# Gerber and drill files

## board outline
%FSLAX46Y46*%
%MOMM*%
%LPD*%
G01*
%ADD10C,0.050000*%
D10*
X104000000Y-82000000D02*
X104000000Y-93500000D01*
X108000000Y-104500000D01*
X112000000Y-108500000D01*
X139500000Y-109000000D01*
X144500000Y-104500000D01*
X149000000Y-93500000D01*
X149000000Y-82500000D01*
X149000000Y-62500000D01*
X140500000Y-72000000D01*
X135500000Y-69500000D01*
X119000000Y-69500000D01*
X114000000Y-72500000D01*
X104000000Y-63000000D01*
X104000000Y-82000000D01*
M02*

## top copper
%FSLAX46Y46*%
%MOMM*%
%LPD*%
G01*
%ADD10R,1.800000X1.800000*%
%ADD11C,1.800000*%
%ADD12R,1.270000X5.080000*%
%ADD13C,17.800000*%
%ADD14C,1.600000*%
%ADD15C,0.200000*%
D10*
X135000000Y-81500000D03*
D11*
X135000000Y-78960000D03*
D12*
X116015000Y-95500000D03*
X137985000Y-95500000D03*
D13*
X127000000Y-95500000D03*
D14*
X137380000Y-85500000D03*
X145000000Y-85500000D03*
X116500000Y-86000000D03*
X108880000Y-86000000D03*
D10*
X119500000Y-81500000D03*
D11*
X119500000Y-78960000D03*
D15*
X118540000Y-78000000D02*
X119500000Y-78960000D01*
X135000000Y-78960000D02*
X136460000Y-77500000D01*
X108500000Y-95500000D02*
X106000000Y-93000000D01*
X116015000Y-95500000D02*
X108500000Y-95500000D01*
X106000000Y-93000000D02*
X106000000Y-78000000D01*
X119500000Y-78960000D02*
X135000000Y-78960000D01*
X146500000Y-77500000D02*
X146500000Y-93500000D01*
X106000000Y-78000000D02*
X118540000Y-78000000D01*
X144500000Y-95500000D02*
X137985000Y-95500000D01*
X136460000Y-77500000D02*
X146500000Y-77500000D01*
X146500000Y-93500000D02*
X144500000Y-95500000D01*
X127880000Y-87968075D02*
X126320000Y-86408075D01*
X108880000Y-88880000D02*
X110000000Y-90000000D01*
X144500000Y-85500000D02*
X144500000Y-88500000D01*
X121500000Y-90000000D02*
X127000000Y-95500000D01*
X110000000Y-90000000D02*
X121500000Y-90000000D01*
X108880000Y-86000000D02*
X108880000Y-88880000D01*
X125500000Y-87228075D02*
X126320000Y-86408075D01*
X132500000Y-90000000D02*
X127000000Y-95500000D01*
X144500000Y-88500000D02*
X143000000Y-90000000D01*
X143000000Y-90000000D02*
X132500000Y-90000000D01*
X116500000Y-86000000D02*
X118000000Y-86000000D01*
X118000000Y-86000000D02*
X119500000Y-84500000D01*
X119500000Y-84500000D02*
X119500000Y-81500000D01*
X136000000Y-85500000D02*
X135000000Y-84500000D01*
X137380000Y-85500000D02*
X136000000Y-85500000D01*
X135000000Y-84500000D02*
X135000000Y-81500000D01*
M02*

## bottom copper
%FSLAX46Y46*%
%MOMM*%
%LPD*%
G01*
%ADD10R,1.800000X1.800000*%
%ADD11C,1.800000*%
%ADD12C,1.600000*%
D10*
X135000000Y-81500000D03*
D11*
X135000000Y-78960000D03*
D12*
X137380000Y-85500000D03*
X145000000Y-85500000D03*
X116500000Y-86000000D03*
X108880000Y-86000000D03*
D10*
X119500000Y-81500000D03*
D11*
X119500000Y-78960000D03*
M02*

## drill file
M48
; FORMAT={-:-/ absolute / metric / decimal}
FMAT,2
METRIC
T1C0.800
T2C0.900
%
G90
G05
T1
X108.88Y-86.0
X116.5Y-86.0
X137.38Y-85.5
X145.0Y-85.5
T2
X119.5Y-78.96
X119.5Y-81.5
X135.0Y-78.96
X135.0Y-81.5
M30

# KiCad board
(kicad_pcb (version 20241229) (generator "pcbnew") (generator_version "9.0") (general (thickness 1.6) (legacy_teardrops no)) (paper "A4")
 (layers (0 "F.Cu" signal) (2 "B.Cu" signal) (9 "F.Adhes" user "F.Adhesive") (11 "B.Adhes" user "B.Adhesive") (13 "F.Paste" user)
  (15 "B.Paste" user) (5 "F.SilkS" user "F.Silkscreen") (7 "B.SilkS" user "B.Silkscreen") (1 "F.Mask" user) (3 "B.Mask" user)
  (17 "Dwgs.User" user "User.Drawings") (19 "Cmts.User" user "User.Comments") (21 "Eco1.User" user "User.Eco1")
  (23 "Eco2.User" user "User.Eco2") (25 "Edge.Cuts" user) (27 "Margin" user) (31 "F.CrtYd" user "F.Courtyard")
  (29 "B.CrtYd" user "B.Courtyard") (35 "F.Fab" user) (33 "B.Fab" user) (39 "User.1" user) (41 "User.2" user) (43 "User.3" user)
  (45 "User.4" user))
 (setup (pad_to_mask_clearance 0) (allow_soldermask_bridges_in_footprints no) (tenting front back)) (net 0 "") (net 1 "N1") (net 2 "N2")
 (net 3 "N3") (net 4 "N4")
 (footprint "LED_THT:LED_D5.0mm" (layer "F.Cu") (at 135 81.5 90)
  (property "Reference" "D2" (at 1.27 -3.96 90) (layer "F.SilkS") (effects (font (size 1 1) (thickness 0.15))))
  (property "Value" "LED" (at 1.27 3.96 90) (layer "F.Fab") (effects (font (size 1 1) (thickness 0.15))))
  (pad "1" thru_hole rect (at 0 0 90) (size 1.8 1.8) (drill 0.9) (layers "*.Cu" "*.Mask") (remove_unused_layers no) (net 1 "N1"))
  (pad "2" thru_hole circle (at 2.54 0 90) (size 1.8 1.8) (drill 0.9) (layers "*.Cu" "*.Mask") (remove_unused_layers no) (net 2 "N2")))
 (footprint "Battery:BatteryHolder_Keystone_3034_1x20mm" (layer "F.Cu") (at 127 95.5)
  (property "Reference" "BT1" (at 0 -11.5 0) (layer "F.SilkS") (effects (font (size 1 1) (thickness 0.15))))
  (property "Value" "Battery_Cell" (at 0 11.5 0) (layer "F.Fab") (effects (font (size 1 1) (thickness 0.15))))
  (pad "1" smd rect (at -10.985 0) (size 1.27 5.08) (layers "F.Cu" "F.Mask" "F.Paste") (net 2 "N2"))
  (pad "1" smd rect (at 10.985 0) (size 1.27 5.08) (layers "F.Cu" "F.Mask" "F.Paste") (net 2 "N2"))
  (pad "2" smd circle (at 0 0) (size 17.8 17.8) (layers "F.Cu" "F.Mask") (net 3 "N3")))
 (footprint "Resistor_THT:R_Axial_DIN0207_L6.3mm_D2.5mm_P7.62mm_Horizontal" (layer "F.Cu") (at 137.38 85.5)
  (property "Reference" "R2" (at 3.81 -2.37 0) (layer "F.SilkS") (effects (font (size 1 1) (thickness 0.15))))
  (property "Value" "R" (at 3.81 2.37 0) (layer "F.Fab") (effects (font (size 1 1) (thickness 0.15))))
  (pad "1" thru_hole circle (at 0 0) (size 1.6 1.6) (drill 0.8) (layers "*.Cu" "*.Mask") (remove_unused_layers no) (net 1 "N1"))
  (pad "2" thru_hole circle (at 7.62 0) (size 1.6 1.6) (drill 0.8) (layers "*.Cu" "*.Mask") (remove_unused_layers no) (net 3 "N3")))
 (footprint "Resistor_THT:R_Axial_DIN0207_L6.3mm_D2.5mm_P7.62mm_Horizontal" (layer "F.Cu") (at 116.5 86 180)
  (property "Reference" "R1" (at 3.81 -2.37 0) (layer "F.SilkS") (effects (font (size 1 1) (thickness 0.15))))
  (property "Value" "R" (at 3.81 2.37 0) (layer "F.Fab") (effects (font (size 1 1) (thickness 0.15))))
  (pad "1" thru_hole circle (at 0 0 180) (size 1.6 1.6) (drill 0.8) (layers "*.Cu" "*.Mask") (remove_unused_layers no) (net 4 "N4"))
  (pad "2" thru_hole circle (at 7.62 0 180) (size 1.6 1.6) (drill 0.8) (layers "*.Cu" "*.Mask") (remove_unused_layers no) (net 3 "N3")))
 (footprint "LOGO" (layer "F.Cu") (at 146 73)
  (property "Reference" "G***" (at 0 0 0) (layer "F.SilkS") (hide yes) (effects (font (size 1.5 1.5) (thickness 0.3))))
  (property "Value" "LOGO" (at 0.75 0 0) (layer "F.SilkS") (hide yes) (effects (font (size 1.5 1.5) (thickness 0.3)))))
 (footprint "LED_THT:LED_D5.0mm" (layer "F.Cu") (at 119.5 81.5 90)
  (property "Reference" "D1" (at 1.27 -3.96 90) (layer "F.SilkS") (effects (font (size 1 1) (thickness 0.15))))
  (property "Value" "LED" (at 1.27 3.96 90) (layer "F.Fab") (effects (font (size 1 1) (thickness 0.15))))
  (pad "1" thru_hole rect (at 0 0 90) (size 1.8 1.8) (drill 0.9) (layers "*.Cu" "*.Mask") (remove_unused_layers no) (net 4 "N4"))
  (pad "2" thru_hole circle (at 2.54 0 90) (size 1.8 1.8) (drill 0.9) (layers "*.Cu" "*.Mask") (remove_unused_layers no) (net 2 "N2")))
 (gr_poly
  (pts (xy 104 82) (xy 104 93.5) (xy 108 104.5) (xy 112 108.5) (xy 139.5 109) (xy 144.5 104.5) (xy 149 93.5) (xy 149 82.5) (xy 149 62.5)
   (xy 140.5 72) (xy 135.5 69.5) (xy 119 69.5) (xy 114 72.5) (xy 104 63))
  (stroke (width 0.05) (type solid)) (fill no) (layer "Edge.Cuts"))
 (segment (start 118.54 78) (end 119.5 78.96) (width 0.2) (layer "F.Cu") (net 2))
 (segment (start 135 78.96) (end 136.46 77.5) (width 0.2) (layer "F.Cu") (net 2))
 (segment (start 108.5 95.5) (end 106 93) (width 0.2) (layer "F.Cu") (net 2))
 (segment (start 116.015 95.5) (end 108.5 95.5) (width 0.2) (layer "F.Cu") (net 2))
 (segment (start 106 93) (end 106 78) (width 0.2) (layer "F.Cu") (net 2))
 (segment (start 119.5 78.96) (end 135 78.96) (width 0.2) (layer "F.Cu") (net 2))
 (segment (start 146.5 77.5) (end 146.5 93.5) (width 0.2) (layer "F.Cu") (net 2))
 (segment (start 106 78) (end 118.54 78) (width 0.2) (layer "F.Cu") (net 2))
 (segment (start 144.5 95.5) (end 137.985 95.5) (width 0.2) (layer "F.Cu") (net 2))
 (segment (start 136.46 77.5) (end 146.5 77.5) (width 0.2) (layer "F.Cu") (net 2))
 (segment (start 146.5 93.5) (end 144.5 95.5) (width 0.2) (layer "F.Cu") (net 2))
 (segment (start 127.88 87.968075) (end 126.32 86.408075) (width 0.2) (layer "F.Cu") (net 3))
 (segment (start 108.88 88.88) (end 110 90) (width 0.2) (layer "F.Cu") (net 3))
 (segment (start 144.5 85.5) (end 144.5 88.5) (width 0.2) (layer "F.Cu") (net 3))
 (segment (start 121.5 90) (end 127 95.5) (width 0.2) (layer "F.Cu") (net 3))
 (segment (start 110 90) (end 121.5 90) (width 0.2) (layer "F.Cu") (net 3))
 (segment (start 108.88 86) (end 108.88 88.88) (width 0.2) (layer "F.Cu") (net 3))
 (segment (start 125.5 87.228075) (end 126.32 86.408075) (width 0.2) (layer "F.Cu") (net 3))
 (segment (start 132.5 90) (end 127 95.5) (width 0.2) (layer "F.Cu") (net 3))
 (segment (start 144.5 88.5) (end 143 90) (width 0.2) (layer "F.Cu") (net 3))
 (segment (start 143 90) (end 132.5 90) (width 0.2) (layer "F.Cu") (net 3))
 (segment (start 116.5 86) (end 118 86) (width 0.2) (layer "F.Cu") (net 4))
 (segment (start 118 86) (end 119.5 84.5) (width 0.2) (layer "F.Cu") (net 4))
 (segment (start 119.5 84.5) (end 119.5 81.5) (width 0.2) (layer "F.Cu") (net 4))
 (segment (start 136 85.5) (end 135 84.5) (width 0.2) (layer "F.Cu") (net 1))
 (segment (start 137.38 85.5) (end 136 85.5) (width 0.2) (layer "F.Cu") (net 1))
 (segment (start 135 84.5) (end 135 81.5) (width 0.2) (layer "F.Cu") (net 1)))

